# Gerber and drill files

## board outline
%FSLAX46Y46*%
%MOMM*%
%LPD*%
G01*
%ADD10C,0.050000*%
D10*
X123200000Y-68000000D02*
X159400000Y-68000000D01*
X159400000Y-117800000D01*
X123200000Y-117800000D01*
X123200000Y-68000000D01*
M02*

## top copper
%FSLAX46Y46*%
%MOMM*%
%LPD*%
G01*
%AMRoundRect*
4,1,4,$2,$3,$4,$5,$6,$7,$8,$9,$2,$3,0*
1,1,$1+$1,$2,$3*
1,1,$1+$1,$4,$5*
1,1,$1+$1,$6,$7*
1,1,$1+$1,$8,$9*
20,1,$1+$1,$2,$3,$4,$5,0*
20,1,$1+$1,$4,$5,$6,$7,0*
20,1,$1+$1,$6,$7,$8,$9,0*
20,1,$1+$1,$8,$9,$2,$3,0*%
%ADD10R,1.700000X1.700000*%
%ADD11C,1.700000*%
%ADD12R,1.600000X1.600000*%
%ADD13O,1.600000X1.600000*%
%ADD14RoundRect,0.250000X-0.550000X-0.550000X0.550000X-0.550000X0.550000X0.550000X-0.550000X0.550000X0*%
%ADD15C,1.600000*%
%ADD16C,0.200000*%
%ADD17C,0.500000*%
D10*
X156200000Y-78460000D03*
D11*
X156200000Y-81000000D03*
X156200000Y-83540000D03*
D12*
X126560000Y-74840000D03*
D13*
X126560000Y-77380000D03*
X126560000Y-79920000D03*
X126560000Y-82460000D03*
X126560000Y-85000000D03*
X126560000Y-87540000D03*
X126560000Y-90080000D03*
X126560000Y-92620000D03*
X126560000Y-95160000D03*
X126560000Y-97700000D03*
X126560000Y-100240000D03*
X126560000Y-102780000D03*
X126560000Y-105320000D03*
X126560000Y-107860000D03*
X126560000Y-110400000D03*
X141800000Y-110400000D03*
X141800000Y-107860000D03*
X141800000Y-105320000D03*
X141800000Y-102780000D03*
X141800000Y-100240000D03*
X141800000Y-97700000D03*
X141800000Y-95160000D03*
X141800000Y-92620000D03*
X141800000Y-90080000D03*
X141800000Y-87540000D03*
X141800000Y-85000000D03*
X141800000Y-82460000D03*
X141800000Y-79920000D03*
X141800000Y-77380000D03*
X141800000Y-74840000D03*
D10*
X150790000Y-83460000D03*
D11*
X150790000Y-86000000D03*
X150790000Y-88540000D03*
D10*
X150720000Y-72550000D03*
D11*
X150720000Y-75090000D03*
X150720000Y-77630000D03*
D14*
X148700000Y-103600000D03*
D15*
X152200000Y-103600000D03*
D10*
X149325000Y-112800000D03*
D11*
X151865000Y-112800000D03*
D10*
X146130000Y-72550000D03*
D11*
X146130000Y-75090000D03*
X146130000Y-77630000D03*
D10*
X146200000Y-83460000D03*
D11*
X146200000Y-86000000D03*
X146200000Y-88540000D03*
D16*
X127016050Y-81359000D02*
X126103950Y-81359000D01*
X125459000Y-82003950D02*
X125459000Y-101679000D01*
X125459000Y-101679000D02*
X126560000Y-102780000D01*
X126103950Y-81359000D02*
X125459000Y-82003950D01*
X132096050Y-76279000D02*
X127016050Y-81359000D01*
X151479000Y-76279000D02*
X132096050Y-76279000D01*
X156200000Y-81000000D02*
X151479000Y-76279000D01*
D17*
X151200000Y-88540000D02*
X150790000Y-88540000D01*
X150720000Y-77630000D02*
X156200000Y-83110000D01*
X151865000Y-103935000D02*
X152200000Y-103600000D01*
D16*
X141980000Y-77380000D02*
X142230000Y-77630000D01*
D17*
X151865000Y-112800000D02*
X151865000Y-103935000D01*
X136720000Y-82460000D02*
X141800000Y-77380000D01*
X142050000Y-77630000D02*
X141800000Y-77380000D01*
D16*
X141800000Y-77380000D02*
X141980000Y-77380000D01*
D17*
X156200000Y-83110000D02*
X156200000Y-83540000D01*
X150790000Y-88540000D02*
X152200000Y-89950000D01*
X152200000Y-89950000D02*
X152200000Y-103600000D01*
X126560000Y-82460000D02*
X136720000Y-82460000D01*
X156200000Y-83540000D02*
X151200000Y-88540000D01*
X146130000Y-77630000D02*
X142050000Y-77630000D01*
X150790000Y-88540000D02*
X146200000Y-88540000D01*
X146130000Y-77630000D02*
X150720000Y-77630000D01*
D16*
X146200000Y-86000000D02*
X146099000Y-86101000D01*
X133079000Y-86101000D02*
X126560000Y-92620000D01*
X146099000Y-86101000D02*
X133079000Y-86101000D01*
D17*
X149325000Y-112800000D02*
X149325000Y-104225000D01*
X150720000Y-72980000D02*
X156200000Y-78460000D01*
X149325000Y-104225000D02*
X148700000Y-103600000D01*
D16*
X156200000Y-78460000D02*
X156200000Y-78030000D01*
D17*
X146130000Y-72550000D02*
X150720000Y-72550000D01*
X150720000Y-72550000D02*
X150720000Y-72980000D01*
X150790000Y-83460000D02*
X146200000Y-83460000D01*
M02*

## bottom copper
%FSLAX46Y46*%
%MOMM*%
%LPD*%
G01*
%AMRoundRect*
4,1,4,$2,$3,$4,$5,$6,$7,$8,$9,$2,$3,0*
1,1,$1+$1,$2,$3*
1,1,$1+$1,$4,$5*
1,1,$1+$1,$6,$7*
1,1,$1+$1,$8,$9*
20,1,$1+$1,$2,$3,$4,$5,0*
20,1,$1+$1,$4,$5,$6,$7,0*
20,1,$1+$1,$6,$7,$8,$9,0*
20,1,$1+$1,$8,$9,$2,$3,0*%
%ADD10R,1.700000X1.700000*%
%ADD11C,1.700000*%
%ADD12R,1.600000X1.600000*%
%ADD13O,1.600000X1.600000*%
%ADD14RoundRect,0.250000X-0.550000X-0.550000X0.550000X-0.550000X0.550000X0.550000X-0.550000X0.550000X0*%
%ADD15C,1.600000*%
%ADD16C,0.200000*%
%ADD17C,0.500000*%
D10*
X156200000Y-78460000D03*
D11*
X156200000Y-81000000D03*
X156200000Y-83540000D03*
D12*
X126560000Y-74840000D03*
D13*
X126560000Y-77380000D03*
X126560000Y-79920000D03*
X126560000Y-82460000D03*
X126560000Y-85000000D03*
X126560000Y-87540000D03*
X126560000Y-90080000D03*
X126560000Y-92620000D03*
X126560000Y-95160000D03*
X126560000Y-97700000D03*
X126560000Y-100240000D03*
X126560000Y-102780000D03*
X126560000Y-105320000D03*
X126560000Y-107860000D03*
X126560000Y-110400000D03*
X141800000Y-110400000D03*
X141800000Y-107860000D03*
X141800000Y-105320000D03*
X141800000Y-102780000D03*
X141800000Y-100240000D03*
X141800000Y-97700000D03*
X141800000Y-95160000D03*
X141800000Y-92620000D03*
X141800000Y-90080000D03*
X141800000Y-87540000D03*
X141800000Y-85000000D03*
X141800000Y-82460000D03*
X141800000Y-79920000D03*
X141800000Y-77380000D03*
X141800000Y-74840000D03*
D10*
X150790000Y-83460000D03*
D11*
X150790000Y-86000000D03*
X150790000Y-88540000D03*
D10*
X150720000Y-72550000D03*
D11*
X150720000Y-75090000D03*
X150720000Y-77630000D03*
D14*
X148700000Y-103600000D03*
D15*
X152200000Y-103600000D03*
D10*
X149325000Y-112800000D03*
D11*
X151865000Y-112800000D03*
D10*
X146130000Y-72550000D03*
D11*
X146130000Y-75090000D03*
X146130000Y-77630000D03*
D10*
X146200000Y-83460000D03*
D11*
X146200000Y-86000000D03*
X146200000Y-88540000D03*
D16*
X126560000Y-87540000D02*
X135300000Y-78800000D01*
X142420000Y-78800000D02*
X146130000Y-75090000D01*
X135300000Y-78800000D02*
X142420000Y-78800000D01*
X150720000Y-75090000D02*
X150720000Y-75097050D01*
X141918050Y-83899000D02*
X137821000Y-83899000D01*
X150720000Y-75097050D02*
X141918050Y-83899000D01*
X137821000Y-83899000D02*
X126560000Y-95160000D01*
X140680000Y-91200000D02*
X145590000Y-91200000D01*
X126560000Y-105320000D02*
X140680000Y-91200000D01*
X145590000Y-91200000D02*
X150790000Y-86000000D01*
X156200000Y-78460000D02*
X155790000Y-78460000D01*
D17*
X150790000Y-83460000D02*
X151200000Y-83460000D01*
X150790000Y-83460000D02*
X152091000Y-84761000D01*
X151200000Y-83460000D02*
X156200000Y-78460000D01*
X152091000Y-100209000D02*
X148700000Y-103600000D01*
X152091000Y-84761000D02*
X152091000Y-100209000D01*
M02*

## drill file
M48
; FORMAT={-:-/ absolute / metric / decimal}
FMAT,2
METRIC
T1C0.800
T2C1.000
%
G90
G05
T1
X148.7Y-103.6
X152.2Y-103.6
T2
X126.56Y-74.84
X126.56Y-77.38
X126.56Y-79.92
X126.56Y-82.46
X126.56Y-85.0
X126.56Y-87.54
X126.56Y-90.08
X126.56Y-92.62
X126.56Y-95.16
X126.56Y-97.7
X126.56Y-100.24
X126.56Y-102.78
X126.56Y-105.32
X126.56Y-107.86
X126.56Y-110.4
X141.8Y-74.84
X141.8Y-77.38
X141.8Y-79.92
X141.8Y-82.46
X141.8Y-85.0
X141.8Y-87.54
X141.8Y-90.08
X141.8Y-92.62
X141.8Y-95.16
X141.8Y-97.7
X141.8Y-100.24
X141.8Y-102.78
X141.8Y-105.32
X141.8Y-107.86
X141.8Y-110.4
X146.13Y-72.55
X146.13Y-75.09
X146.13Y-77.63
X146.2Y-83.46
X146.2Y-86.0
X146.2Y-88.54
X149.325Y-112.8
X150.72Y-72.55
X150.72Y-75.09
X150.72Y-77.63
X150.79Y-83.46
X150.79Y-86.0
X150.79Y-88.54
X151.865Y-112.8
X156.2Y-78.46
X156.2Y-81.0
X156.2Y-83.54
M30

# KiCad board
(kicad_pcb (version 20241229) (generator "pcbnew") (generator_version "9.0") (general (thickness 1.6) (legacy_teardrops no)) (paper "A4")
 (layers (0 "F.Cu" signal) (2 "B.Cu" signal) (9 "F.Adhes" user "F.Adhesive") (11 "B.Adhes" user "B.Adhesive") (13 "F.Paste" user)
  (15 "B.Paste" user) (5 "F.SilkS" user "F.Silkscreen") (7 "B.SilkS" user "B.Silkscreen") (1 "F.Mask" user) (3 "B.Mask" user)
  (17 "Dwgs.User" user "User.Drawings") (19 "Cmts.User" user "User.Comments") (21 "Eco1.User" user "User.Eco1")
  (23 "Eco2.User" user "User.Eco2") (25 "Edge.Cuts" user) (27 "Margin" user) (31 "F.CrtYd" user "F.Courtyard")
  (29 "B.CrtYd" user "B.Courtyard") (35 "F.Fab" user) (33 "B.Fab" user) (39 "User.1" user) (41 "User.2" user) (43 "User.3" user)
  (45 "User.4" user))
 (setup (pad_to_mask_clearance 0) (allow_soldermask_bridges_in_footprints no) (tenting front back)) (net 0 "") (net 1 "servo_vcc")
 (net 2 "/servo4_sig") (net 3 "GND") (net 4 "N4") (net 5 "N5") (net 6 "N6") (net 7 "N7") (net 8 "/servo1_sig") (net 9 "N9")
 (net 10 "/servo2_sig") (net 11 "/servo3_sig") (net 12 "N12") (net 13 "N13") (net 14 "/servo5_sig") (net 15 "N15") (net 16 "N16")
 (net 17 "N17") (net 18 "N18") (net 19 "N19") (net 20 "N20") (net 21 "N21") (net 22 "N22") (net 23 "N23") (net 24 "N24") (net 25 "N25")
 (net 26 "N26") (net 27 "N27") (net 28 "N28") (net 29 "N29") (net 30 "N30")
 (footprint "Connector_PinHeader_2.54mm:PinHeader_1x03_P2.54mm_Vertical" (layer "F.Cu") (at 156.2 78.46)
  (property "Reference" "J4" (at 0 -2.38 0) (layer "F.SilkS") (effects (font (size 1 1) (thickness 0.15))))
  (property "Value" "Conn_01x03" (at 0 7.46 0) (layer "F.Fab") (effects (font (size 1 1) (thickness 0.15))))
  (pad "1" thru_hole rect (at 0 0) (size 1.7 1.7) (drill 1) (layers "*.Cu" "*.Mask") (remove_unused_layers no) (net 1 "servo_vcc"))
  (pad "2" thru_hole circle (at 0 2.54) (size 1.7 1.7) (drill 1) (layers "*.Cu" "*.Mask") (remove_unused_layers no) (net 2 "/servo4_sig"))
  (pad "3" thru_hole circle (at 0 5.08) (size 1.7 1.7) (drill 1) (layers "*.Cu" "*.Mask") (remove_unused_layers no) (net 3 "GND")))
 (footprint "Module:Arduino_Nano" (layer "F.Cu") (at 126.56 74.84)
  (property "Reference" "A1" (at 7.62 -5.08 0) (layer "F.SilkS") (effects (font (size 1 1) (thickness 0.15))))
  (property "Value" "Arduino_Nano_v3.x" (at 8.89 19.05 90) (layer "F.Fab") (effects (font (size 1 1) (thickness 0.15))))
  (pad "1" thru_hole rect (at 0 0) (size 1.6 1.6) (drill 1) (layers "*.Cu" "*.Mask") (remove_unused_layers no) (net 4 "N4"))
  (pad "2" thru_hole oval (at 0 2.54) (size 1.6 1.6) (drill 1) (layers "*.Cu" "*.Mask") (remove_unused_layers no) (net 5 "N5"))
  (pad "3" thru_hole oval (at 0 5.08) (size 1.6 1.6) (drill 1) (layers "*.Cu" "*.Mask") (remove_unused_layers no) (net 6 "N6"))
  (pad "4" thru_hole oval (at 0 7.62) (size 1.6 1.6) (drill 1) (layers "*.Cu" "*.Mask") (remove_unused_layers no) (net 3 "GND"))
  (pad "5" thru_hole oval (at 0 10.16) (size 1.6 1.6) (drill 1) (layers "*.Cu" "*.Mask") (remove_unused_layers no) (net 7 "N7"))
  (pad "6" thru_hole oval (at 0 12.7) (size 1.6 1.6) (drill 1) (layers "*.Cu" "*.Mask") (remove_unused_layers no) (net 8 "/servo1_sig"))
  (pad "7" thru_hole oval (at 0 15.24) (size 1.6 1.6) (drill 1) (layers "*.Cu" "*.Mask") (remove_unused_layers no) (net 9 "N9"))
  (pad "8" thru_hole oval (at 0 17.78) (size 1.6 1.6) (drill 1) (layers "*.Cu" "*.Mask") (remove_unused_layers no) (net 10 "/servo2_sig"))
  (pad "9" thru_hole oval (at 0 20.32) (size 1.6 1.6) (drill 1) (layers "*.Cu" "*.Mask") (remove_unused_layers no) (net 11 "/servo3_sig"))
  (pad "10" thru_hole oval (at 0 22.86) (size 1.6 1.6) (drill 1) (layers "*.Cu" "*.Mask") (remove_unused_layers no) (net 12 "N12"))
  (pad "11" thru_hole oval (at 0 25.4) (size 1.6 1.6) (drill 1) (layers "*.Cu" "*.Mask") (remove_unused_layers no) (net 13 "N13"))
  (pad "12" thru_hole oval (at 0 27.94) (size 1.6 1.6) (drill 1) (layers "*.Cu" "*.Mask") (remove_unused_layers no) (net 2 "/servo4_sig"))
  (pad "13" thru_hole oval (at 0 30.48) (size 1.6 1.6) (drill 1) (layers "*.Cu" "*.Mask") (remove_unused_layers no) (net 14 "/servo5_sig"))
  (pad "14" thru_hole oval (at 0 33.02) (size 1.6 1.6) (drill 1) (layers "*.Cu" "*.Mask") (remove_unused_layers no) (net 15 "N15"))
  (pad "15" thru_hole oval (at 0 35.56) (size 1.6 1.6) (drill 1) (layers "*.Cu" "*.Mask") (remove_unused_layers no) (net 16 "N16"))
  (pad "16" thru_hole oval (at 15.24 35.56) (size 1.6 1.6) (drill 1) (layers "*.Cu" "*.Mask") (remove_unused_layers no) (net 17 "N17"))
  (pad "17" thru_hole oval (at 15.24 33.02) (size 1.6 1.6) (drill 1) (layers "*.Cu" "*.Mask") (remove_unused_layers no) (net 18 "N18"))
  (pad "18" thru_hole oval (at 15.24 30.48) (size 1.6 1.6) (drill 1) (layers "*.Cu" "*.Mask") (remove_unused_layers no) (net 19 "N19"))
  (pad "19" thru_hole oval (at 15.24 27.94) (size 1.6 1.6) (drill 1) (layers "*.Cu" "*.Mask") (remove_unused_layers no) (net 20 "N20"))
  (pad "20" thru_hole oval (at 15.24 25.4) (size 1.6 1.6) (drill 1) (layers "*.Cu" "*.Mask") (remove_unused_layers no) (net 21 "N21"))
  (pad "21" thru_hole oval (at 15.24 22.86) (size 1.6 1.6) (drill 1) (layers "*.Cu" "*.Mask") (remove_unused_layers no) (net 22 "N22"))
  (pad "22" thru_hole oval (at 15.24 20.32) (size 1.6 1.6) (drill 1) (layers "*.Cu" "*.Mask") (remove_unused_layers no) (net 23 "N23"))
  (pad "23" thru_hole oval (at 15.24 17.78) (size 1.6 1.6) (drill 1) (layers "*.Cu" "*.Mask") (remove_unused_layers no) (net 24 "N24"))
  (pad "24" thru_hole oval (at 15.24 15.24) (size 1.6 1.6) (drill 1) (layers "*.Cu" "*.Mask") (remove_unused_layers no) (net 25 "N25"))
  (pad "25" thru_hole oval (at 15.24 12.7) (size 1.6 1.6) (drill 1) (layers "*.Cu" "*.Mask") (remove_unused_layers no) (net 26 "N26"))
  (pad "26" thru_hole oval (at 15.24 10.16) (size 1.6 1.6) (drill 1) (layers "*.Cu" "*.Mask") (remove_unused_layers no) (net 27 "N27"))
  (pad "27" thru_hole oval (at 15.24 7.62) (size 1.6 1.6) (drill 1) (layers "*.Cu" "*.Mask") (remove_unused_layers no) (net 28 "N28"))
  (pad "28" thru_hole oval (at 15.24 5.08) (size 1.6 1.6) (drill 1) (layers "*.Cu" "*.Mask") (remove_unused_layers no) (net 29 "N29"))
  (pad "29" thru_hole oval (at 15.24 2.54) (size 1.6 1.6) (drill 1) (layers "*.Cu" "*.Mask") (remove_unused_layers no) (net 3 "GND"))
  (pad "30" thru_hole oval (at 15.24 0) (size 1.6 1.6) (drill 1) (layers "*.Cu" "*.Mask") (remove_unused_layers no) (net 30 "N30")))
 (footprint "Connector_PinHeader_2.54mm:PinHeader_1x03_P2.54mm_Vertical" (layer "F.Cu") (at 150.79 83.46)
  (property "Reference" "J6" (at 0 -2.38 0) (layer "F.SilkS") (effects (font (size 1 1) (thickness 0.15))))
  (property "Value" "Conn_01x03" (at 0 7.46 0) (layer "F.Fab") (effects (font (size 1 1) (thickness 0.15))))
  (pad "1" thru_hole rect (at 0 0) (size 1.7 1.7) (drill 1) (layers "*.Cu" "*.Mask") (remove_unused_layers no) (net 1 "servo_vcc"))
  (pad "2" thru_hole circle (at 0 2.54) (size 1.7 1.7) (drill 1) (layers "*.Cu" "*.Mask") (remove_unused_layers no) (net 14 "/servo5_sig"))
  (pad "3" thru_hole circle (at 0 5.08) (size 1.7 1.7) (drill 1) (layers "*.Cu" "*.Mask") (remove_unused_layers no) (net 3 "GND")))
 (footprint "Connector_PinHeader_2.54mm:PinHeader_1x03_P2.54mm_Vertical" (layer "F.Cu") (at 150.72 72.55)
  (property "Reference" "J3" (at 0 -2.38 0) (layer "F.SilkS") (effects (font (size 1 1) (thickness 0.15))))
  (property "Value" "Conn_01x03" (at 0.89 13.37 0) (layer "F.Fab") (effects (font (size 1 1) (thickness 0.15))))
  (pad "1" thru_hole rect (at 0 0) (size 1.7 1.7) (drill 1) (layers "*.Cu" "*.Mask") (remove_unused_layers no) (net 1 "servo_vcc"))
  (pad "2" thru_hole circle (at 0 2.54) (size 1.7 1.7) (drill 1) (layers "*.Cu" "*.Mask") (remove_unused_layers no) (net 11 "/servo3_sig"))
  (pad "3" thru_hole circle (at 0 5.08) (size 1.7 1.7) (drill 1) (layers "*.Cu" "*.Mask") (remove_unused_layers no) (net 3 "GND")))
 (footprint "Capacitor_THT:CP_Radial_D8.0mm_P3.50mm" (layer "F.Cu") (at 148.7 103.6)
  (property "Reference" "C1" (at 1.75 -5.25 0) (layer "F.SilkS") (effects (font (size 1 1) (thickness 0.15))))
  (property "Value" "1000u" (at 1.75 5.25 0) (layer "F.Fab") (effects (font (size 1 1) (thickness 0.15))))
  (pad "1" thru_hole roundrect (at 0 0) (size 1.6 1.6) (drill 0.8) (layers "*.Cu" "*.Mask") (remove_unused_layers no)
   (roundrect_rratio 0.15625) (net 1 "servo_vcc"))
  (pad "2" thru_hole circle (at 3.5 0) (size 1.6 1.6) (drill 0.8) (layers "*.Cu" "*.Mask") (remove_unused_layers no) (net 3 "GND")))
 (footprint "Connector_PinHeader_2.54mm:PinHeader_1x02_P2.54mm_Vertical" (layer "F.Cu") (at 149.325 112.8 90)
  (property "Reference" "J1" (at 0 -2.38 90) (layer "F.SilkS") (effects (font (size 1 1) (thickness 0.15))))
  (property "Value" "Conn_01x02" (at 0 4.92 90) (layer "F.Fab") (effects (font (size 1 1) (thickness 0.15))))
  (pad "1" thru_hole rect (at 0 0 90) (size 1.7 1.7) (drill 1) (layers "*.Cu" "*.Mask") (remove_unused_layers no) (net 1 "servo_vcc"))
  (pad "2" thru_hole circle (at 0 2.54 90) (size 1.7 1.7) (drill 1) (layers "*.Cu" "*.Mask") (remove_unused_layers no) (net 3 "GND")))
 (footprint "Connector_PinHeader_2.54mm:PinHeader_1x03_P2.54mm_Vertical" (layer "F.Cu") (at 146.13 72.55)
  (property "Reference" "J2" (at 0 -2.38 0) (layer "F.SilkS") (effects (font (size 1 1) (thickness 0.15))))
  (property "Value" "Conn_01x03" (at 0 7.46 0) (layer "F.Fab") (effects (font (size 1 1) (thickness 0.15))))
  (pad "1" thru_hole rect (at 0 0) (size 1.7 1.7) (drill 1) (layers "*.Cu" "*.Mask") (remove_unused_layers no) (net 1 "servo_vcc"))
  (pad "2" thru_hole circle (at 0 2.54) (size 1.7 1.7) (drill 1) (layers "*.Cu" "*.Mask") (remove_unused_layers no) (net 8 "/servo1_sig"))
  (pad "3" thru_hole circle (at 0 5.08) (size 1.7 1.7) (drill 1) (layers "*.Cu" "*.Mask") (remove_unused_layers no) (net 3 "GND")))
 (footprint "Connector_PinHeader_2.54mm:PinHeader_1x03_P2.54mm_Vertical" (layer "F.Cu") (at 146.2 83.46)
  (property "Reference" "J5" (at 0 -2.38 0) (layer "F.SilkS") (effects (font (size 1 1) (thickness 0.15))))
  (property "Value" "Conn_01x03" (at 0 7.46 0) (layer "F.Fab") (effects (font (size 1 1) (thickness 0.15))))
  (pad "1" thru_hole rect (at 0 0) (size 1.7 1.7) (drill 1) (layers "*.Cu" "*.Mask") (remove_unused_layers no) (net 1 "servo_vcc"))
  (pad "2" thru_hole circle (at 0 2.54) (size 1.7 1.7) (drill 1) (layers "*.Cu" "*.Mask") (remove_unused_layers no) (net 10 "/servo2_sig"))
  (pad "3" thru_hole circle (at 0 5.08) (size 1.7 1.7) (drill 1) (layers "*.Cu" "*.Mask") (remove_unused_layers no) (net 3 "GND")))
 (gr_rect (start 123.2 68) (end 159.4 117.8) (stroke (width 0.05) (type default)) (fill no) (layer "Edge.Cuts"))
 (segment (start 127.01605 81.359) (end 126.10395 81.359) (width 0.2) (layer "F.Cu") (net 2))
 (segment (start 125.459 82.00395) (end 125.459 101.679) (width 0.2) (layer "F.Cu") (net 2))
 (segment (start 125.459 101.679) (end 126.56 102.78) (width 0.2) (layer "F.Cu") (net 2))
 (segment (start 126.10395 81.359) (end 125.459 82.00395) (width 0.2) (layer "F.Cu") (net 2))
 (segment (start 132.09605 76.279) (end 127.01605 81.359) (width 0.2) (layer "F.Cu") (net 2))
 (segment (start 151.479 76.279) (end 132.09605 76.279) (width 0.2) (layer "F.Cu") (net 2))
 (segment (start 156.2 81) (end 151.479 76.279) (width 0.2) (layer "F.Cu") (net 2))
 (segment (start 151.2 88.54) (end 150.79 88.54) (width 0.5) (layer "F.Cu") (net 3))
 (segment (start 150.72 77.63) (end 156.2 83.11) (width 0.5) (layer "F.Cu") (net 3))
 (segment (start 151.865 103.935) (end 152.2 103.6) (width 0.5) (layer "F.Cu") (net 3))
 (segment (start 141.98 77.38) (end 142.23 77.63) (width 0.2) (layer "F.Cu") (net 3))
 (segment (start 151.865 112.8) (end 151.865 103.935) (width 0.5) (layer "F.Cu") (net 3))
 (segment (start 136.72 82.46) (end 141.8 77.38) (width 0.5) (layer "F.Cu") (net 3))
 (segment (start 142.05 77.63) (end 141.8 77.38) (width 0.5) (layer "F.Cu") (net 3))
 (segment (start 141.8 77.38) (end 141.98 77.38) (width 0.2) (layer "F.Cu") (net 3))
 (segment (start 156.2 83.11) (end 156.2 83.54) (width 0.5) (layer "F.Cu") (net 3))
 (segment (start 150.79 88.54) (end 152.2 89.95) (width 0.5) (layer "F.Cu") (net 3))
 (segment (start 152.2 89.95) (end 152.2 103.6) (width 0.5) (layer "F.Cu") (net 3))
 (segment (start 126.56 82.46) (end 136.72 82.46) (width 0.5) (layer "F.Cu") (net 3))
 (segment (start 156.2 83.54) (end 151.2 88.54) (width 0.5) (layer "F.Cu") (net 3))
 (segment (start 146.13 77.63) (end 142.05 77.63) (width 0.5) (layer "F.Cu") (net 3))
 (segment (start 150.79 88.54) (end 146.2 88.54) (width 0.5) (layer "F.Cu") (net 3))
 (segment (start 146.13 77.63) (end 150.72 77.63) (width 0.5) (layer "F.Cu") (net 3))
 (segment (start 126.56 87.54) (end 135.3 78.8) (width 0.2) (layer "B.Cu") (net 8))
 (segment (start 142.42 78.8) (end 146.13 75.09) (width 0.2) (layer "B.Cu") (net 8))
 (segment (start 135.3 78.8) (end 142.42 78.8) (width 0.2) (layer "B.Cu") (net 8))
 (segment (start 146.2 86) (end 146.099 86.101) (width 0.2) (layer "F.Cu") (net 10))
 (segment (start 133.079 86.101) (end 126.56 92.62) (width 0.2) (layer "F.Cu") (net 10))
 (segment (start 146.099 86.101) (end 133.079 86.101) (width 0.2) (layer "F.Cu") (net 10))
 (segment (start 150.72 75.09) (end 150.72 75.09705) (width 0.2) (layer "B.Cu") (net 11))
 (segment (start 141.91805 83.899) (end 137.821 83.899) (width 0.2) (layer "B.Cu") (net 11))
 (segment (start 150.72 75.09705) (end 141.91805 83.899) (width 0.2) (layer "B.Cu") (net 11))
 (segment (start 137.821 83.899) (end 126.56 95.16) (width 0.2) (layer "B.Cu") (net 11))
 (segment (start 140.68 91.2) (end 145.59 91.2) (width 0.2) (layer "B.Cu") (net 14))
 (segment (start 126.56 105.32) (end 140.68 91.2) (width 0.2) (layer "B.Cu") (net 14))
 (segment (start 145.59 91.2) (end 150.79 86) (width 0.2) (layer "B.Cu") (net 14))
 (segment (start 149.325 112.8) (end 149.325 104.225) (width 0.5) (layer "F.Cu") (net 1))
 (segment (start 150.72 72.98) (end 156.2 78.46) (width 0.5) (layer "F.Cu") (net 1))
 (segment (start 149.325 104.225) (end 148.7 103.6) (width 0.5) (layer "F.Cu") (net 1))
 (segment (start 156.2 78.46) (end 156.2 78.03) (width 0.2) (layer "F.Cu") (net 1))
 (segment (start 146.13 72.55) (end 150.72 72.55) (width 0.5) (layer "F.Cu") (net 1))
 (segment (start 150.72 72.55) (end 150.72 72.98) (width 0.5) (layer "F.Cu") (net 1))
 (segment (start 150.79 83.46) (end 146.2 83.46) (width 0.5) (layer "F.Cu") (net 1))
 (segment (start 156.2 78.46) (end 155.79 78.46) (width 0.2) (layer "B.Cu") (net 1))
 (segment (start 150.79 83.46) (end 151.2 83.46) (width 0.5) (layer "B.Cu") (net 1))
 (segment (start 150.79 83.46) (end 152.091 84.761) (width 0.5) (layer "B.Cu") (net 1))
 (segment (start 151.2 83.46) (end 156.2 78.46) (width 0.5) (layer "B.Cu") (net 1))
 (segment (start 152.091 100.209) (end 148.7 103.6) (width 0.5) (layer "B.Cu") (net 1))
 (segment (start 152.091 84.761) (end 152.091 100.209) (width 0.5) (layer "B.Cu") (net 1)))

